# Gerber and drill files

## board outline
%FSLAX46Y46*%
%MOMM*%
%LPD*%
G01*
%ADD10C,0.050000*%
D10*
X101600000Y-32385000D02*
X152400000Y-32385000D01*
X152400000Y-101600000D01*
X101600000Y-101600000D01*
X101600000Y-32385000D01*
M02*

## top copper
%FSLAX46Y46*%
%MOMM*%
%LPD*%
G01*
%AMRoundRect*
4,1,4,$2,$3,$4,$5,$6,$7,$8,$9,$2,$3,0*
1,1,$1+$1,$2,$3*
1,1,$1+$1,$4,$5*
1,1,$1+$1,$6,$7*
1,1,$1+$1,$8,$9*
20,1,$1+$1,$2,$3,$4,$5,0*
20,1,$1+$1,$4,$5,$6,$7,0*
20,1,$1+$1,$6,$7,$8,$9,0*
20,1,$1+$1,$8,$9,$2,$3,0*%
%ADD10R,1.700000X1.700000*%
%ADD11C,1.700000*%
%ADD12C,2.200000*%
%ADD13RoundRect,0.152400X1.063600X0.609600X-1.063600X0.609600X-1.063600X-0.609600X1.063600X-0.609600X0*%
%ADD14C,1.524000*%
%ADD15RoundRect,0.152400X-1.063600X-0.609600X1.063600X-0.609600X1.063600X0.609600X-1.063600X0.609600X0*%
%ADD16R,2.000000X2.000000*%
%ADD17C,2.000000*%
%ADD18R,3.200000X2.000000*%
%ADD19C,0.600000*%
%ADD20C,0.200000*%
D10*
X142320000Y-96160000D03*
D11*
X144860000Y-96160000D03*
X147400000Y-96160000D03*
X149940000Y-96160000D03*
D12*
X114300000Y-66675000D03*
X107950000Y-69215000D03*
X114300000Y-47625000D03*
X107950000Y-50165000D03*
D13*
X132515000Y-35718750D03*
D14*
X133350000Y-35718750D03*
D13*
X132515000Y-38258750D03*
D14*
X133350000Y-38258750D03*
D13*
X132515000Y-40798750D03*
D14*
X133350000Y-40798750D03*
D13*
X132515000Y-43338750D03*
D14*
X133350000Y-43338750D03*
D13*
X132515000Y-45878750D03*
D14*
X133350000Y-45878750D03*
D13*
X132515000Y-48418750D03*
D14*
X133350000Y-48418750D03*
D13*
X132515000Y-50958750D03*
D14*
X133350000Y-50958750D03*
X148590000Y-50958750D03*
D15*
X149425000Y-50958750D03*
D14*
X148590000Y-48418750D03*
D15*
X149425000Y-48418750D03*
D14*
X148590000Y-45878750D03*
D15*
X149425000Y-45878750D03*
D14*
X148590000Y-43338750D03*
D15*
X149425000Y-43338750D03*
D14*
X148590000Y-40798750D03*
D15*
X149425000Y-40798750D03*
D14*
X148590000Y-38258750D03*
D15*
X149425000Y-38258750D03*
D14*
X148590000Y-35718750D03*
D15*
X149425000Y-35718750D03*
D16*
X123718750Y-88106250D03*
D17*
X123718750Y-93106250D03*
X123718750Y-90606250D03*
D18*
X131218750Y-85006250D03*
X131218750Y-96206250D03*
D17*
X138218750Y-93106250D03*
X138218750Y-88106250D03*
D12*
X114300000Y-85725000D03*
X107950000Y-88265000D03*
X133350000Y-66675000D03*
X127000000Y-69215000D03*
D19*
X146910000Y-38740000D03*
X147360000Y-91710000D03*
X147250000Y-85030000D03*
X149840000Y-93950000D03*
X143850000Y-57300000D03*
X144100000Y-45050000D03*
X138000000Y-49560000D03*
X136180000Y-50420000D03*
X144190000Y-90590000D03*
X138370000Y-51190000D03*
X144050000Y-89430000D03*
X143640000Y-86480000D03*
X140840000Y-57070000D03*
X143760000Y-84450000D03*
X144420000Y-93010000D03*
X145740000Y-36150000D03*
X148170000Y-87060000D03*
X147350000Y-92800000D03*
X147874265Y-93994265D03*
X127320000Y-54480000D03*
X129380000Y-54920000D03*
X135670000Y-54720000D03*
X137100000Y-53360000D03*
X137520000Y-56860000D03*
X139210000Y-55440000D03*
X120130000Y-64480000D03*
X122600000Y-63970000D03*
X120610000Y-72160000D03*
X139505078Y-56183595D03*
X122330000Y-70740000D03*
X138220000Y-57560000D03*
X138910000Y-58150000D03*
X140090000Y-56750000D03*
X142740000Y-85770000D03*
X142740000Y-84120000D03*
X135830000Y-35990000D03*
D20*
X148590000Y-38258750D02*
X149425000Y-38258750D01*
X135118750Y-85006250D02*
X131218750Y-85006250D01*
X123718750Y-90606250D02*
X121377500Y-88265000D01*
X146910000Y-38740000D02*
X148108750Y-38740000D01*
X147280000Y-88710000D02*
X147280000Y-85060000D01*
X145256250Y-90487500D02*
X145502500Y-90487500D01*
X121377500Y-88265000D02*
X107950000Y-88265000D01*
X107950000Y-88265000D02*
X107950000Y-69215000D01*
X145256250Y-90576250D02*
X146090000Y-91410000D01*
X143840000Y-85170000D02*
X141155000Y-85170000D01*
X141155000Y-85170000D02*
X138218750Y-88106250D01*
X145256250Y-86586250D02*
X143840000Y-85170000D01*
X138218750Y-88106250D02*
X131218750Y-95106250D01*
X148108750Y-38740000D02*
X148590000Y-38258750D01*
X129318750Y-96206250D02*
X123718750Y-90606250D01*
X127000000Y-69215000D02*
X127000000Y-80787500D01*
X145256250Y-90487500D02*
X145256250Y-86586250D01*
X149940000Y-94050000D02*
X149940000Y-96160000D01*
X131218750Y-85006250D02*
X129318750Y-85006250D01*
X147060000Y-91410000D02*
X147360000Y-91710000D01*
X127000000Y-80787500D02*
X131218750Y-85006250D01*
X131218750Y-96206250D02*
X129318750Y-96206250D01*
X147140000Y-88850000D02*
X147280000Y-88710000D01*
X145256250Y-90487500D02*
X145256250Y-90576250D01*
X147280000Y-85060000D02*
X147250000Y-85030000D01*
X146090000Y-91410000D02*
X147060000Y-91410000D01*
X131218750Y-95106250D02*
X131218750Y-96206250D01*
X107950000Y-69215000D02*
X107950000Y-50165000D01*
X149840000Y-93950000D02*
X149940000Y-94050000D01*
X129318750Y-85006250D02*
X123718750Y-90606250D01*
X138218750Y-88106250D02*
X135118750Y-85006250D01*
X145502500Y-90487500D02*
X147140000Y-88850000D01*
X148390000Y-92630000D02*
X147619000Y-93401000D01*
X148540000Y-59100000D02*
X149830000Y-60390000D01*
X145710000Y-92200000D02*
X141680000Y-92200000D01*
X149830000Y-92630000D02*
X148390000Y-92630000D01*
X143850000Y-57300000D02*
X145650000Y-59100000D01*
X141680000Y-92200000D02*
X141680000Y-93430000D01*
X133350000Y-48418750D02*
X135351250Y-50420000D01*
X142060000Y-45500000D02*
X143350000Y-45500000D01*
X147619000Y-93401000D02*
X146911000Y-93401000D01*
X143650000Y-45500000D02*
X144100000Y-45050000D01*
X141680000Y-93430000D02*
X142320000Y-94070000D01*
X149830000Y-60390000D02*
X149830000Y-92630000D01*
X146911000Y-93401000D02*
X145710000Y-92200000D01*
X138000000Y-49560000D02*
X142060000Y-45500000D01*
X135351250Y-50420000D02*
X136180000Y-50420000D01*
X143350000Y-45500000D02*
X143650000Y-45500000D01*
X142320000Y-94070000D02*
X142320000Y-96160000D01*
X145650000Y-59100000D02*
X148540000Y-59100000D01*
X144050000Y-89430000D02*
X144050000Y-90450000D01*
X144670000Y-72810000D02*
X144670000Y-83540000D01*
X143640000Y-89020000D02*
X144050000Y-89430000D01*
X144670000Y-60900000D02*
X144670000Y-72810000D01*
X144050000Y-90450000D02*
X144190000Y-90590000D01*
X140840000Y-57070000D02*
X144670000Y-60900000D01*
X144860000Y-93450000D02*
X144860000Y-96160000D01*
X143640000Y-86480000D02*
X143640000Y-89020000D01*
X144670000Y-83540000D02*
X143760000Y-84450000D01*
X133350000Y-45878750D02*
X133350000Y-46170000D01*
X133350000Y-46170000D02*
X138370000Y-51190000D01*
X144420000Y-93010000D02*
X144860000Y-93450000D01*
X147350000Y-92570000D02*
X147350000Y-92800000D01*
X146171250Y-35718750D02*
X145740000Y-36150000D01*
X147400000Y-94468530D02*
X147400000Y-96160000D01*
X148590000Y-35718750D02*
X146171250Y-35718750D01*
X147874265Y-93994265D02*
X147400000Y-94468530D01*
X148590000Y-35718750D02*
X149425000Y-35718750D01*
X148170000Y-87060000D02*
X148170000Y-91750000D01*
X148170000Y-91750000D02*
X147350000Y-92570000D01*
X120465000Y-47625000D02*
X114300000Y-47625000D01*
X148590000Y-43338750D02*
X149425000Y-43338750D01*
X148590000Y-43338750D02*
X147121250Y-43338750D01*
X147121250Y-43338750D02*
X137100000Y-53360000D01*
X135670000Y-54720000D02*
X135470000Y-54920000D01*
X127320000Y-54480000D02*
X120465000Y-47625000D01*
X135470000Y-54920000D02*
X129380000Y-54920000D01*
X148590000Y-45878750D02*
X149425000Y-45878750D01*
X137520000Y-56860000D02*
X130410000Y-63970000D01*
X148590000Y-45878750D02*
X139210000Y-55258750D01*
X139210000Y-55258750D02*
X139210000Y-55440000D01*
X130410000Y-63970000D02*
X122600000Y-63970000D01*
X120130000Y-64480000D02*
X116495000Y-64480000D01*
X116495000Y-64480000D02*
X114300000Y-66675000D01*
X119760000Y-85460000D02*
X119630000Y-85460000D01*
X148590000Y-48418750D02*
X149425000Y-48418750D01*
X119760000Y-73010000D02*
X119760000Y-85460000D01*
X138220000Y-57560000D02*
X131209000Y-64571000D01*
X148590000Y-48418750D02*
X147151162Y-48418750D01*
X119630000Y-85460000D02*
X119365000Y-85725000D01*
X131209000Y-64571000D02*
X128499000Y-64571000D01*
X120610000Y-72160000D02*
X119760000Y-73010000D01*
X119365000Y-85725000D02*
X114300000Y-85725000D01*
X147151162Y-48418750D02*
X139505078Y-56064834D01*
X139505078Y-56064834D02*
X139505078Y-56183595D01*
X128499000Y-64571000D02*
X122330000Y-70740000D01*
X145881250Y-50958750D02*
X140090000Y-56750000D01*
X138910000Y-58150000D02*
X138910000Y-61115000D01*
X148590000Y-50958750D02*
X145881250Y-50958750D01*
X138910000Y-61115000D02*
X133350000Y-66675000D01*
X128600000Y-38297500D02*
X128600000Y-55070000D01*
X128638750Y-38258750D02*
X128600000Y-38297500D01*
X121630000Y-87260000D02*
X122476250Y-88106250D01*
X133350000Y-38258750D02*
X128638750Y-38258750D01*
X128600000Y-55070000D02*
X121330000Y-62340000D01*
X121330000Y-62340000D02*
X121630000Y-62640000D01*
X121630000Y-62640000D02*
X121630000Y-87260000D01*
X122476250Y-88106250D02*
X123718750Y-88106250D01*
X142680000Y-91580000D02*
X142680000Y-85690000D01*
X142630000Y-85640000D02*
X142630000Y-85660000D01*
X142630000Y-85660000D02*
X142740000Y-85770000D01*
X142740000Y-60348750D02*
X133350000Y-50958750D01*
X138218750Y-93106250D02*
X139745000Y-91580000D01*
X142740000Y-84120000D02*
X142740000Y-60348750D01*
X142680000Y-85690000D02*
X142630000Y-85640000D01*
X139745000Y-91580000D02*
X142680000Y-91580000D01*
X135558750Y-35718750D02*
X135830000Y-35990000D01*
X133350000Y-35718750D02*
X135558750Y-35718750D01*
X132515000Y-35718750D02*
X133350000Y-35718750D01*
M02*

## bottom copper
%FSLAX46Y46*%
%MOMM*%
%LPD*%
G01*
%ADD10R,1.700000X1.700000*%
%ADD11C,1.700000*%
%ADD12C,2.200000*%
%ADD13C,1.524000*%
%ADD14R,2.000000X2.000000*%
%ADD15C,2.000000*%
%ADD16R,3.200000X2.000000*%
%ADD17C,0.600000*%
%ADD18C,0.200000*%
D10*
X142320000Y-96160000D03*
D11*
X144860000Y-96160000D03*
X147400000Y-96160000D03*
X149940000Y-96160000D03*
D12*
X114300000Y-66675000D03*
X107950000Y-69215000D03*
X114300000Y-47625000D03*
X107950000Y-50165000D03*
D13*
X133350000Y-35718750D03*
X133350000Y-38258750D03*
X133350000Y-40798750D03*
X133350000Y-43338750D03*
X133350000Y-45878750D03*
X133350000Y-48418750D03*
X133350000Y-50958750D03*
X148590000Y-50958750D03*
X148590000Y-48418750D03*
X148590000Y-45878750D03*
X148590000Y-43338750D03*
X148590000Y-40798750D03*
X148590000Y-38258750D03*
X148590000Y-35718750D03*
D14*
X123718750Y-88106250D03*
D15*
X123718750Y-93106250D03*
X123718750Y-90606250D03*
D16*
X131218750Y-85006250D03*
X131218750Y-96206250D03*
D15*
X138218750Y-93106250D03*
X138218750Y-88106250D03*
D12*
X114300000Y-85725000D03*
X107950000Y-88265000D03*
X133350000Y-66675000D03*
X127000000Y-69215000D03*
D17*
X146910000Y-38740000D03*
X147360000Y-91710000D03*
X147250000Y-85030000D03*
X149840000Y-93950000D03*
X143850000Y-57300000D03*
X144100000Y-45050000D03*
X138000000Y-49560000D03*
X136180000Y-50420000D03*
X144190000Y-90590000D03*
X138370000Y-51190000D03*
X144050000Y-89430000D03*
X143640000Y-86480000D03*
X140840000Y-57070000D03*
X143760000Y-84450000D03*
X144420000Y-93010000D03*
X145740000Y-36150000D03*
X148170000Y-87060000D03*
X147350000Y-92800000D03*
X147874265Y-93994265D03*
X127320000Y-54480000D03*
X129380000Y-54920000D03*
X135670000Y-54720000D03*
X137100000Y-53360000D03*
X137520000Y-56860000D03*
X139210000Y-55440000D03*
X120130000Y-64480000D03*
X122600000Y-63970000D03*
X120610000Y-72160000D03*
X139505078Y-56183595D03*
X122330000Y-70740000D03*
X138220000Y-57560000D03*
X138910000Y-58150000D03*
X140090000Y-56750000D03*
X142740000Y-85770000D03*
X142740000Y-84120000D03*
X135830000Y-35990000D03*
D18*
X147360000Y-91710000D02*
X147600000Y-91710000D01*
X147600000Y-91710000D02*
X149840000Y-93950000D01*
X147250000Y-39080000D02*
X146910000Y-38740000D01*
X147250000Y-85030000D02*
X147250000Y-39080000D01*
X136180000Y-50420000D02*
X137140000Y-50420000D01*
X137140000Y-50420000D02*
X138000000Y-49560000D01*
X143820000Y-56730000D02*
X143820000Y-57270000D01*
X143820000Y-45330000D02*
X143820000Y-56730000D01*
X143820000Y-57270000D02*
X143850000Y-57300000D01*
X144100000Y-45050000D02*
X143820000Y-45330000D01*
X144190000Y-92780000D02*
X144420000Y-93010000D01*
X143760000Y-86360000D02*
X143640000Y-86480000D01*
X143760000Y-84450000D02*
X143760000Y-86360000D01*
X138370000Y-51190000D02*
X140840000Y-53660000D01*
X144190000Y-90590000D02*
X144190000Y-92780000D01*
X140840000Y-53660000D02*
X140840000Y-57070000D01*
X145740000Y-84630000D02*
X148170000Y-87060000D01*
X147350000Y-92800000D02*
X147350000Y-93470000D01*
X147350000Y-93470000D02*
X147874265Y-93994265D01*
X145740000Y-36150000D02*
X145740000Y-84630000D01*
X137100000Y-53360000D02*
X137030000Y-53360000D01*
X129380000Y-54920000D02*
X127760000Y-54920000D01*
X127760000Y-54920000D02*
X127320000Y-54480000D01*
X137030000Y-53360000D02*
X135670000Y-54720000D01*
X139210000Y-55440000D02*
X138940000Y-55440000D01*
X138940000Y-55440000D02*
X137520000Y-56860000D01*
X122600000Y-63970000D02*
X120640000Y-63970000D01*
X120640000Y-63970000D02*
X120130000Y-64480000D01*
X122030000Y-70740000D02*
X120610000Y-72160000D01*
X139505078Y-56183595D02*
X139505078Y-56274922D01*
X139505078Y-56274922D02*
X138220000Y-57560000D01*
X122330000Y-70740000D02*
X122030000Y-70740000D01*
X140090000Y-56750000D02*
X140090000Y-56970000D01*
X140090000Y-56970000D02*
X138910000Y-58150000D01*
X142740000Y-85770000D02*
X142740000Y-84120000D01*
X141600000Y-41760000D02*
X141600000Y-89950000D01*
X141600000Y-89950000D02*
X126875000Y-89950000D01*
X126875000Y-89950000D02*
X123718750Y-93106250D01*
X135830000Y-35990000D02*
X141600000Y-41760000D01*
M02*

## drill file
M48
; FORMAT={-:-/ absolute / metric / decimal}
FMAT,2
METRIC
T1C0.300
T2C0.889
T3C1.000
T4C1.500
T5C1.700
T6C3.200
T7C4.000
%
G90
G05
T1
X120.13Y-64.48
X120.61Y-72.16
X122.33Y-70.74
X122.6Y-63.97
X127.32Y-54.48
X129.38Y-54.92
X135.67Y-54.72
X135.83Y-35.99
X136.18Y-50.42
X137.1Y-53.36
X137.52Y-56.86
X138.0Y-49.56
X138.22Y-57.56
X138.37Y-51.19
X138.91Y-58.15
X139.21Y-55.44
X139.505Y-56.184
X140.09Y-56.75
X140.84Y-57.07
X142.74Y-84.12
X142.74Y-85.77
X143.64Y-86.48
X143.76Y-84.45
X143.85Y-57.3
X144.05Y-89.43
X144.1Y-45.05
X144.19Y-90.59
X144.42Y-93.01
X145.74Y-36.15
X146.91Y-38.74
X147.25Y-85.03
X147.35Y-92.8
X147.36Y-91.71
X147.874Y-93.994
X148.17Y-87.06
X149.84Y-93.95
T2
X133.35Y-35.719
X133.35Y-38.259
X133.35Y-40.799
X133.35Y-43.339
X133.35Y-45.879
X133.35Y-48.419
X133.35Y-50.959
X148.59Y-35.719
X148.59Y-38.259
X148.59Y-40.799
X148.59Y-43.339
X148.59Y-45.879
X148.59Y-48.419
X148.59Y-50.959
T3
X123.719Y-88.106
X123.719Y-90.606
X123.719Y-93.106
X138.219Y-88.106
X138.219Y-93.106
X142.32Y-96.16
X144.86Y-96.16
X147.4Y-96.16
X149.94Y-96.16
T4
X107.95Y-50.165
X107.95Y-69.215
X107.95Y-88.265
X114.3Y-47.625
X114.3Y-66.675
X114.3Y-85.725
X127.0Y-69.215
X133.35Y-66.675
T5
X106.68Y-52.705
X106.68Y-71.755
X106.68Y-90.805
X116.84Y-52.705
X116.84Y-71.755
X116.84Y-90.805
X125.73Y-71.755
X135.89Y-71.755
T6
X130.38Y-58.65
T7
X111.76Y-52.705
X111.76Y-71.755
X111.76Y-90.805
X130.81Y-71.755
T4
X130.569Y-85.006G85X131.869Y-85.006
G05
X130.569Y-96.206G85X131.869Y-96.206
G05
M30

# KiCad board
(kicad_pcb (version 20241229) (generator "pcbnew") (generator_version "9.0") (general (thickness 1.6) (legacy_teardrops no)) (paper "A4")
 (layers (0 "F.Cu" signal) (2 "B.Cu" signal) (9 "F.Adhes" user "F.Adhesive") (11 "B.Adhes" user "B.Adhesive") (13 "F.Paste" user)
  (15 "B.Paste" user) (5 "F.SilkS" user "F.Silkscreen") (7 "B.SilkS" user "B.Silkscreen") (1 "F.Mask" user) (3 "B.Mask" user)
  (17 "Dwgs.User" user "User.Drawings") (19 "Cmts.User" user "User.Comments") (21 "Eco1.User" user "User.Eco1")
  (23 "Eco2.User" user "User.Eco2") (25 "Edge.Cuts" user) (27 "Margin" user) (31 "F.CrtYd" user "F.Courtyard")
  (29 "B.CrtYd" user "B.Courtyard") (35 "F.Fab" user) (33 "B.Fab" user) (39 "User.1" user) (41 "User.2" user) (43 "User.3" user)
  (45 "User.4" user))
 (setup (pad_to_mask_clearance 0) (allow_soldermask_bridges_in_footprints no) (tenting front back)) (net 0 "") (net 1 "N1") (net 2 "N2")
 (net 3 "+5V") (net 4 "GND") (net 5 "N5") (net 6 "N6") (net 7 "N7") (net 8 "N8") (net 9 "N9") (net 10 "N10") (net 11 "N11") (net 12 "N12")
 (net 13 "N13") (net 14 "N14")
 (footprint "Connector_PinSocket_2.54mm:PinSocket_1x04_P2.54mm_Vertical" (layer "F.Cu") (at 142.32 96.16 90)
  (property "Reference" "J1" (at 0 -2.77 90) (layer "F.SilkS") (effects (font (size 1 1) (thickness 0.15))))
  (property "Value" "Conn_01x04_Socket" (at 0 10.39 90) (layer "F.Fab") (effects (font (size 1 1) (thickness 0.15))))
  (pad "1" thru_hole rect (at 0 0 90) (size 1.7 1.7) (drill 1) (layers "*.Cu" "*.Mask") (remove_unused_layers no) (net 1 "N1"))
  (pad "2" thru_hole circle (at 0 2.54 90) (size 1.7 1.7) (drill 1) (layers "*.Cu" "*.Mask") (remove_unused_layers no) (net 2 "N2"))
  (pad "3" thru_hole circle (at 0 5.08 90) (size 1.7 1.7) (drill 1) (layers "*.Cu" "*.Mask") (remove_unused_layers no) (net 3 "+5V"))
  (pad "4" thru_hole circle (at 0 7.62 90) (size 1.7 1.7) (drill 1) (layers "*.Cu" "*.Mask") (remove_unused_layers no) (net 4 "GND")))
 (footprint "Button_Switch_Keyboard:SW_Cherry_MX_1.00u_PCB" (layer "F.Cu") (at 114.3 66.675)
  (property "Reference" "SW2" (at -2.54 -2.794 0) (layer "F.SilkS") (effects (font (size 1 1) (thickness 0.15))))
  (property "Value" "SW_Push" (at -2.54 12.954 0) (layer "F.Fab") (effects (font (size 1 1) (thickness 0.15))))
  (pad "" np_thru_hole circle (at -7.62 5.08) (size 1.7 1.7) (drill 1.7) (layers "*.Cu" "*.Mask"))
  (pad "" np_thru_hole circle (at -2.54 5.08) (size 4 4) (drill 4) (layers "*.Cu" "*.Mask"))
  (pad "" np_thru_hole circle (at 2.54 5.08) (size 1.7 1.7) (drill 1.7) (layers "*.Cu" "*.Mask"))
  (pad "1" thru_hole circle (at 0 0) (size 2.2 2.2) (drill 1.5) (layers "*.Cu" "*.Mask") (remove_unused_layers no) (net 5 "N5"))
  (pad "2" thru_hole circle (at -6.35 2.54) (size 2.2 2.2) (drill 1.5) (layers "*.Cu" "*.Mask") (remove_unused_layers no) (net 4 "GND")))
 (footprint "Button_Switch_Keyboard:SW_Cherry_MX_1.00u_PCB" (layer "F.Cu") (at 114.3 47.625)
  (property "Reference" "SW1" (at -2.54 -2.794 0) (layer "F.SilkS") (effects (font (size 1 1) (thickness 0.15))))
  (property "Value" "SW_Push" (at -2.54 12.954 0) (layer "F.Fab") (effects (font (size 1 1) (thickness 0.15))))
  (pad "" np_thru_hole circle (at -7.62 5.08) (size 1.7 1.7) (drill 1.7) (layers "*.Cu" "*.Mask"))
  (pad "" np_thru_hole circle (at -2.54 5.08) (size 4 4) (drill 4) (layers "*.Cu" "*.Mask"))
  (pad "" np_thru_hole circle (at 2.54 5.08) (size 1.7 1.7) (drill 1.7) (layers "*.Cu" "*.Mask"))
  (pad "1" thru_hole circle (at 0 0) (size 2.2 2.2) (drill 1.5) (layers "*.Cu" "*.Mask") (remove_unused_layers no) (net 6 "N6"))
  (pad "2" thru_hole circle (at -6.35 2.54) (size 2.2 2.2) (drill 1.5) (layers "*.Cu" "*.Mask") (remove_unused_layers no) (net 4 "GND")))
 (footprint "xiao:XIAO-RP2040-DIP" (layer "F.Cu") (at 140.97 43.33875)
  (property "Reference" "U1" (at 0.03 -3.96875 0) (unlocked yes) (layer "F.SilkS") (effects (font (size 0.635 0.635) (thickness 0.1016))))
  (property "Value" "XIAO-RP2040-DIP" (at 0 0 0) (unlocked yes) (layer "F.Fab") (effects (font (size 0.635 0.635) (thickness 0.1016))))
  (pad "1" smd roundrect (at -8.455 -7.62 180) (size 2.432 1.524) (layers "F.Cu" "F.Mask") (roundrect_rratio 0.1) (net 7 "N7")
   (thermal_bridge_angle 45))
  (pad "1" thru_hole circle (at -7.62 -7.62 180) (size 1.524 1.524) (drill 0.889) (layers "*.Cu" "*.Mask") (remove_unused_layers no)
   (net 7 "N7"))
  (pad "2" smd roundrect (at -8.455 -5.08 180) (size 2.432 1.524) (layers "F.Cu" "F.Mask") (roundrect_rratio 0.1) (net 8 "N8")
   (thermal_bridge_angle 45))
  (pad "2" thru_hole circle (at -7.62 -5.08 180) (size 1.524 1.524) (drill 0.889) (layers "*.Cu" "*.Mask") (remove_unused_layers no)
   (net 8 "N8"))
  (pad "3" smd roundrect (at -8.455 -2.54 180) (size 2.432 1.524) (layers "F.Cu" "F.Mask") (roundrect_rratio 0.1) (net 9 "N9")
   (thermal_bridge_angle 45))
  (pad "3" thru_hole circle (at -7.62 -2.54 180) (size 1.524 1.524) (drill 0.889) (layers "*.Cu" "*.Mask") (remove_unused_layers no)
   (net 9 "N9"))
  (pad "4" smd roundrect (at -8.455 0 180) (size 2.432 1.524) (layers "F.Cu" "F.Mask") (roundrect_rratio 0.1) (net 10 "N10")
   (thermal_bridge_angle 45))
  (pad "4" thru_hole circle (at -7.62 0 180) (size 1.524 1.524) (drill 0.889) (layers "*.Cu" "*.Mask") (remove_unused_layers no)
   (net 10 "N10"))
  (pad "5" smd roundrect (at -8.455 2.54 180) (size 2.432 1.524) (layers "F.Cu" "F.Mask") (roundrect_rratio 0.1) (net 2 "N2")
   (thermal_bridge_angle 45))
  (pad "5" thru_hole circle (at -7.62 2.54 180) (size 1.524 1.524) (drill 0.889) (layers "*.Cu" "*.Mask") (remove_unused_layers no)
   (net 2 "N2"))
  (pad "6" smd roundrect (at -8.455 5.08 180) (size 2.432 1.524) (layers "F.Cu" "F.Mask") (roundrect_rratio 0.1) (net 1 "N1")
   (thermal_bridge_angle 45))
  (pad "6" thru_hole circle (at -7.62 5.08 180) (size 1.524 1.524) (drill 0.889) (layers "*.Cu" "*.Mask") (remove_unused_layers no)
   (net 1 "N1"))
  (pad "7" smd roundrect (at -8.455 7.62 180) (size 2.432 1.524) (layers "F.Cu" "F.Mask") (roundrect_rratio 0.1) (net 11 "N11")
   (thermal_bridge_angle 45))
  (pad "7" thru_hole circle (at -7.62 7.62 180) (size 1.524 1.524) (drill 0.889) (layers "*.Cu" "*.Mask") (remove_unused_layers no)
   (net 11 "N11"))
  (pad "8" thru_hole circle (at 7.62 7.62) (size 1.524 1.524) (drill 0.889) (layers "*.Cu" "*.Mask") (remove_unused_layers no)
   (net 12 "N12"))
  (pad "8" smd roundrect (at 8.455 7.62) (size 2.432 1.524) (layers "F.Cu" "F.Mask") (roundrect_rratio 0.1) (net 12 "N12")
   (thermal_bridge_angle 45))
  (pad "9" thru_hole circle (at 7.62 5.08) (size 1.524 1.524) (drill 0.889) (layers "*.Cu" "*.Mask") (remove_unused_layers no)
   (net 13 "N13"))
  (pad "9" smd roundrect (at 8.455 5.08) (size 2.432 1.524) (layers "F.Cu" "F.Mask") (roundrect_rratio 0.1) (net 13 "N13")
   (thermal_bridge_angle 45))
  (pad "10" thru_hole circle (at 7.62 2.54) (size 1.524 1.524) (drill 0.889) (layers "*.Cu" "*.Mask") (remove_unused_layers no) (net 5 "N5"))
  (pad "10" smd roundrect (at 8.455 2.54) (size 2.432 1.524) (layers "F.Cu" "F.Mask") (roundrect_rratio 0.1) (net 5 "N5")
   (thermal_bridge_angle 45))
  (pad "11" thru_hole circle (at 7.62 0) (size 1.524 1.524) (drill 0.889) (layers "*.Cu" "*.Mask") (remove_unused_layers no) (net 6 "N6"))
  (pad "11" smd roundrect (at 8.455 0) (size 2.432 1.524) (layers "F.Cu" "F.Mask") (roundrect_rratio 0.1) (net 6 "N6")
   (thermal_bridge_angle 45))
  (pad "12" thru_hole circle (at 7.62 -2.54) (size 1.524 1.524) (drill 0.889) (layers "*.Cu" "*.Mask") (remove_unused_layers no)
   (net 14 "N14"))
  (pad "12" smd roundrect (at 8.455 -2.54) (size 2.432 1.524) (layers "F.Cu" "F.Mask") (roundrect_rratio 0.1) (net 14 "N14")
   (thermal_bridge_angle 45))
  (pad "13" thru_hole circle (at 7.62 -5.08) (size 1.524 1.524) (drill 0.889) (layers "*.Cu" "*.Mask") (remove_unused_layers no)
   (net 4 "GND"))
  (pad "13" smd roundrect (at 8.455 -5.08) (size 2.432 1.524) (layers "F.Cu" "F.Mask") (roundrect_rratio 0.1) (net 4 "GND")
   (thermal_bridge_angle 45))
  (pad "14" thru_hole circle (at 7.62 -7.62) (size 1.524 1.524) (drill 0.889) (layers "*.Cu" "*.Mask") (remove_unused_layers no)
   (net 3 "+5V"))
  (pad "14" smd roundrect (at 8.455 -7.62) (size 2.432 1.524) (layers "F.Cu" "F.Mask") (roundrect_rratio 0.1) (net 3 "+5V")
   (thermal_bridge_angle 45)))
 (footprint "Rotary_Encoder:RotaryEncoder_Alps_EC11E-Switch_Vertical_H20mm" (layer "F.Cu") (at 123.71875 88.10625)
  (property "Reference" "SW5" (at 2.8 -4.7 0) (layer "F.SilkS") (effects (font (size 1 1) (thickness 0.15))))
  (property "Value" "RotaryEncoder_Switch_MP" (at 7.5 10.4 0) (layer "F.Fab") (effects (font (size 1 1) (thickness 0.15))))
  (pad "A" thru_hole rect (at 0 0) (size 2 2) (drill 1) (layers "*.Cu" "*.Mask") (remove_unused_layers no) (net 8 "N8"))
  (pad "B" thru_hole circle (at 0 5) (size 2 2) (drill 1) (layers "*.Cu" "*.Mask") (remove_unused_layers no) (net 7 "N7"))
  (pad "C" thru_hole circle (at 0 2.5) (size 2 2) (drill 1) (layers "*.Cu" "*.Mask") (remove_unused_layers no) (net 4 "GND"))
  (pad "MP" thru_hole rect (at 7.5 -3.1) (size 3.2 2) (drill oval 2.8 1.5) (layers "*.Cu" "*.Mask") (remove_unused_layers no) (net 4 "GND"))
  (pad "MP" thru_hole rect (at 7.5 8.1) (size 3.2 2) (drill oval 2.8 1.5) (layers "*.Cu" "*.Mask") (remove_unused_layers no) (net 4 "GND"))
  (pad "S1" thru_hole circle (at 14.5 5) (size 2 2) (drill 1) (layers "*.Cu" "*.Mask") (remove_unused_layers no) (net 11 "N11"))
  (pad "S2" thru_hole circle (at 14.5 0) (size 2 2) (drill 1) (layers "*.Cu" "*.Mask") (remove_unused_layers no) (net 4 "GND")))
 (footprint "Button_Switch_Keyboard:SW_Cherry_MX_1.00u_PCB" (layer "F.Cu") (at 114.3 85.725)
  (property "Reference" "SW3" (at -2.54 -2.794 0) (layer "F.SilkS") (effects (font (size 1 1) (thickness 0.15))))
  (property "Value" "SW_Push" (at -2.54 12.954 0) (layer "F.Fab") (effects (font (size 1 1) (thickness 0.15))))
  (pad "" np_thru_hole circle (at -7.62 5.08) (size 1.7 1.7) (drill 1.7) (layers "*.Cu" "*.Mask"))
  (pad "" np_thru_hole circle (at -2.54 5.08) (size 4 4) (drill 4) (layers "*.Cu" "*.Mask"))
  (pad "" np_thru_hole circle (at 2.54 5.08) (size 1.7 1.7) (drill 1.7) (layers "*.Cu" "*.Mask"))
  (pad "1" thru_hole circle (at 0 0) (size 2.2 2.2) (drill 1.5) (layers "*.Cu" "*.Mask") (remove_unused_layers no) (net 13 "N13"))
  (pad "2" thru_hole circle (at -6.35 2.54) (size 2.2 2.2) (drill 1.5) (layers "*.Cu" "*.Mask") (remove_unused_layers no) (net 4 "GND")))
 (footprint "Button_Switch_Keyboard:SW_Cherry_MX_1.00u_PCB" (layer "F.Cu") (at 133.35 66.675)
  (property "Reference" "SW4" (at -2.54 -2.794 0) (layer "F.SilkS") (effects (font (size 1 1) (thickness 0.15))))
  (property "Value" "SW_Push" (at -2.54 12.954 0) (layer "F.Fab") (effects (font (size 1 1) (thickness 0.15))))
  (pad "" np_thru_hole circle (at -7.62 5.08) (size 1.7 1.7) (drill 1.7) (layers "*.Cu" "*.Mask"))
  (pad "" np_thru_hole circle (at -2.54 5.08) (size 4 4) (drill 4) (layers "*.Cu" "*.Mask"))
  (pad "" np_thru_hole circle (at 2.54 5.08) (size 1.7 1.7) (drill 1.7) (layers "*.Cu" "*.Mask"))
  (pad "1" thru_hole circle (at 0 0) (size 2.2 2.2) (drill 1.5) (layers "*.Cu" "*.Mask") (remove_unused_layers no) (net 12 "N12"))
  (pad "2" thru_hole circle (at -6.35 2.54) (size 2.2 2.2) (drill 1.5) (layers "*.Cu" "*.Mask") (remove_unused_layers no) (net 4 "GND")))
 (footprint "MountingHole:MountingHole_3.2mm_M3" (layer "F.Cu") (at 130.38 58.65)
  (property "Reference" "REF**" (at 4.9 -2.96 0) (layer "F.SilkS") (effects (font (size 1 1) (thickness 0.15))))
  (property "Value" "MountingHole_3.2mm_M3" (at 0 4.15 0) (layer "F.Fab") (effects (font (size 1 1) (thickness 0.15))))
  (pad "" np_thru_hole circle (at 0 0) (size 3.2 3.2) (drill 3.2) (layers "*.Cu" "*.Mask")))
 (gr_rect (start 101.6 32.385) (end 152.4 101.6) (stroke (width 0.05) (type default)) (fill no) (layer "Edge.Cuts"))
 (segment (start 148.59 38.25875) (end 149.425 38.25875) (width 0.2) (layer "F.Cu") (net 4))
 (segment (start 135.11875 85.00625) (end 131.21875 85.00625) (width 0.2) (layer "F.Cu") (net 4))
 (segment (start 123.71875 90.60625) (end 121.3775 88.265) (width 0.2) (layer "F.Cu") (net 4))
 (segment (start 146.91 38.74) (end 148.10875 38.74) (width 0.2) (layer "F.Cu") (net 4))
 (segment (start 147.28 88.71) (end 147.28 85.06) (width 0.2) (layer "F.Cu") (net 4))
 (segment (start 145.25625 90.4875) (end 145.5025 90.4875) (width 0.2) (layer "F.Cu") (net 4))
 (segment (start 121.3775 88.265) (end 107.95 88.265) (width 0.2) (layer "F.Cu") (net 4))
 (segment (start 107.95 88.265) (end 107.95 69.215) (width 0.2) (layer "F.Cu") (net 4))
 (segment (start 145.25625 90.57625) (end 146.09 91.41) (width 0.2) (layer "F.Cu") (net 4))
 (segment (start 143.84 85.17) (end 141.155 85.17) (width 0.2) (layer "F.Cu") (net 4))
 (segment (start 141.155 85.17) (end 138.21875 88.10625) (width 0.2) (layer "F.Cu") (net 4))
 (segment (start 145.25625 86.58625) (end 143.84 85.17) (width 0.2) (layer "F.Cu") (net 4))
 (segment (start 138.21875 88.10625) (end 131.21875 95.10625) (width 0.2) (layer "F.Cu") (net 4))
 (segment (start 148.10875 38.74) (end 148.59 38.25875) (width 0.2) (layer "F.Cu") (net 4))
 (segment (start 129.31875 96.20625) (end 123.71875 90.60625) (width 0.2) (layer "F.Cu") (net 4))
 (segment (start 127 69.215) (end 127 80.7875) (width 0.2) (layer "F.Cu") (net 4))
 (segment (start 145.25625 90.4875) (end 145.25625 86.58625) (width 0.2) (layer "F.Cu") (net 4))
 (segment (start 149.94 94.05) (end 149.94 96.16) (width 0.2) (layer "F.Cu") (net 4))
 (segment (start 131.21875 85.00625) (end 129.31875 85.00625) (width 0.2) (layer "F.Cu") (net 4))
 (segment (start 147.06 91.41) (end 147.36 91.71) (width 0.2) (layer "F.Cu") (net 4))
 (segment (start 127 80.7875) (end 131.21875 85.00625) (width 0.2) (layer "F.Cu") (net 4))
 (segment (start 131.21875 96.20625) (end 129.31875 96.20625) (width 0.2) (layer "F.Cu") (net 4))
 (segment (start 147.14 88.85) (end 147.28 88.71) (width 0.2) (layer "F.Cu") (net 4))
 (segment (start 145.25625 90.4875) (end 145.25625 90.57625) (width 0.2) (layer "F.Cu") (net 4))
 (segment (start 147.28 85.06) (end 147.25 85.03) (width 0.2) (layer "F.Cu") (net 4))
 (segment (start 146.09 91.41) (end 147.06 91.41) (width 0.2) (layer "F.Cu") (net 4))
 (segment (start 131.21875 95.10625) (end 131.21875 96.20625) (width 0.2) (layer "F.Cu") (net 4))
 (segment (start 107.95 69.215) (end 107.95 50.165) (width 0.2) (layer "F.Cu") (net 4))
 (segment (start 149.84 93.95) (end 149.94 94.05) (width 0.2) (layer "F.Cu") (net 4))
 (segment (start 129.31875 85.00625) (end 123.71875 90.60625) (width 0.2) (layer "F.Cu") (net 4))
 (segment (start 138.21875 88.10625) (end 135.11875 85.00625) (width 0.2) (layer "F.Cu") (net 4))
 (segment (start 145.5025 90.4875) (end 147.14 88.85) (width 0.2) (layer "F.Cu") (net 4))
 (via (at 146.91 38.74) (size 0.6) (drill 0.3) (layers "F.Cu" "B.Cu") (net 4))
 (via (at 147.36 91.71) (size 0.6) (drill 0.3) (layers "F.Cu" "B.Cu") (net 4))
 (via (at 147.25 85.03) (size 0.6) (drill 0.3) (layers "F.Cu" "B.Cu") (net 4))
 (via (at 149.84 93.95) (size 0.6) (drill 0.3) (layers "F.Cu" "B.Cu") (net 4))
 (segment (start 147.36 91.71) (end 147.6 91.71) (width 0.2) (layer "B.Cu") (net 4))
 (segment (start 147.6 91.71) (end 149.84 93.95) (width 0.2) (layer "B.Cu") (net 4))
 (segment (start 147.25 39.08) (end 146.91 38.74) (width 0.2) (layer "B.Cu") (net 4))
 (segment (start 147.25 85.03) (end 147.25 39.08) (width 0.2) (layer "B.Cu") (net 4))
 (segment (start 148.39 92.63) (end 147.619 93.401) (width 0.2) (layer "F.Cu") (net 1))
 (segment (start 148.54 59.1) (end 149.83 60.39) (width 0.2) (layer "F.Cu") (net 1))
 (segment (start 145.71 92.2) (end 141.68 92.2) (width 0.2) (layer "F.Cu") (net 1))
 (segment (start 149.83 92.63) (end 148.39 92.63) (width 0.2) (layer "F.Cu") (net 1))
 (segment (start 143.85 57.3) (end 145.65 59.1) (width 0.2) (layer "F.Cu") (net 1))
 (segment (start 141.68 92.2) (end 141.68 93.43) (width 0.2) (layer "F.Cu") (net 1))
 (segment (start 133.35 48.41875) (end 135.35125 50.42) (width 0.2) (layer "F.Cu") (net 1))
 (segment (start 142.06 45.5) (end 143.35 45.5) (width 0.2) (layer "F.Cu") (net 1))
 (segment (start 147.619 93.401) (end 146.911 93.401) (width 0.2) (layer "F.Cu") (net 1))
 (segment (start 143.65 45.5) (end 144.1 45.05) (width 0.2) (layer "F.Cu") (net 1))
 (segment (start 141.68 93.43) (end 142.32 94.07) (width 0.2) (layer "F.Cu") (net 1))
 (segment (start 149.83 60.39) (end 149.83 92.63) (width 0.2) (layer "F.Cu") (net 1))
 (segment (start 146.911 93.401) (end 145.71 92.2) (width 0.2) (layer "F.Cu") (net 1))
 (segment (start 138 49.56) (end 142.06 45.5) (width 0.2) (layer "F.Cu") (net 1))
 (segment (start 135.35125 50.42) (end 136.18 50.42) (width 0.2) (layer "F.Cu") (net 1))
 (segment (start 143.35 45.5) (end 143.65 45.5) (width 0.2) (layer "F.Cu") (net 1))
 (segment (start 142.32 94.07) (end 142.32 96.16) (width 0.2) (layer "F.Cu") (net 1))
 (segment (start 145.65 59.1) (end 148.54 59.1) (width 0.2) (layer "F.Cu") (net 1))
 (via (at 143.85 57.3) (size 0.6) (drill 0.3) (layers "F.Cu" "B.Cu") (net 1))
 (via (at 144.1 45.05) (size 0.6) (drill 0.3) (layers "F.Cu" "B.Cu") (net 1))
 (via (at 138 49.56) (size 0.6) (drill 0.3) (layers "F.Cu" "B.Cu") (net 1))
 (via (at 136.18 50.42) (size 0.6) (drill 0.3) (layers "F.Cu" "B.Cu") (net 1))
 (segment (start 136.18 50.42) (end 137.14 50.42) (width 0.2) (layer "B.Cu") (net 1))
 (segment (start 137.14 50.42) (end 138 49.56) (width 0.2) (layer "B.Cu") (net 1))
 (segment (start 143.82 56.73) (end 143.82 57.27) (width 0.2) (layer "B.Cu") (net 1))
 (segment (start 143.82 45.33) (end 143.82 56.73) (width 0.2) (layer "B.Cu") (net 1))
 (segment (start 143.82 57.27) (end 143.85 57.3) (width 0.2) (layer "B.Cu") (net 1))
 (segment (start 144.1 45.05) (end 143.82 45.33) (width 0.2) (layer "B.Cu") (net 1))
 (segment (start 144.05 89.43) (end 144.05 90.45) (width 0.2) (layer "F.Cu") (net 2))
 (segment (start 144.67 72.81) (end 144.67 83.54) (width 0.2) (layer "F.Cu") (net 2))
 (segment (start 143.64 89.02) (end 144.05 89.43) (width 0.2) (layer "F.Cu") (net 2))
 (segment (start 144.67 60.9) (end 144.67 72.81) (width 0.2) (layer "F.Cu") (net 2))
 (segment (start 144.05 90.45) (end 144.19 90.59) (width 0.2) (layer "F.Cu") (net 2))
 (segment (start 140.84 57.07) (end 144.67 60.9) (width 0.2) (layer "F.Cu") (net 2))
 (segment (start 144.86 93.45) (end 144.86 96.16) (width 0.2) (layer "F.Cu") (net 2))
 (segment (start 143.64 86.48) (end 143.64 89.02) (width 0.2) (layer "F.Cu") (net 2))
 (segment (start 144.67 83.54) (end 143.76 84.45) (width 0.2) (layer "F.Cu") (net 2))
 (segment (start 133.35 45.87875) (end 133.35 46.17) (width 0.2) (layer "F.Cu") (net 2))
 (segment (start 133.35 46.17) (end 138.37 51.19) (width 0.2) (layer "F.Cu") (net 2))
 (segment (start 144.42 93.01) (end 144.86 93.45) (width 0.2) (layer "F.Cu") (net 2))
 (via (at 144.19 90.59) (size 0.6) (drill 0.3) (layers "F.Cu" "B.Cu") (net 2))
 (via (at 138.37 51.19) (size 0.6) (drill 0.3) (layers "F.Cu" "B.Cu") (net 2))
 (via (at 144.05 89.43) (size 0.6) (drill 0.3) (layers "F.Cu" "B.Cu") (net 2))
 (via (at 143.64 86.48) (size 0.6) (drill 0.3) (layers "F.Cu" "B.Cu") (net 2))
 (via (at 140.84 57.07) (size 0.6) (drill 0.3) (layers "F.Cu" "B.Cu") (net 2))
 (via (at 143.76 84.45) (size 0.6) (drill 0.3) (layers "F.Cu" "B.Cu") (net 2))
 (via (at 144.42 93.01) (size 0.6) (drill 0.3) (layers "F.Cu" "B.Cu") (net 2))
 (segment (start 144.19 92.78) (end 144.42 93.01) (width 0.2) (layer "B.Cu") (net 2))
 (segment (start 143.76 86.36) (end 143.64 86.48) (width 0.2) (layer "B.Cu") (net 2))
 (segment (start 143.76 84.45) (end 143.76 86.36) (width 0.2) (layer "B.Cu") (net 2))
 (segment (start 138.37 51.19) (end 140.84 53.66) (width 0.2) (layer "B.Cu") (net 2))
 (segment (start 144.19 90.59) (end 144.19 92.78) (width 0.2) (layer "B.Cu") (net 2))
 (segment (start 140.84 53.66) (end 140.84 57.07) (width 0.2) (layer "B.Cu") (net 2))
 (segment (start 147.35 92.57) (end 147.35 92.8) (width 0.2) (layer "F.Cu") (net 3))
 (segment (start 146.17125 35.71875) (end 145.74 36.15) (width 0.2) (layer "F.Cu") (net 3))
 (segment (start 147.4 94.46853) (end 147.4 96.16) (width 0.2) (layer "F.Cu") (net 3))
 (segment (start 148.59 35.71875) (end 146.17125 35.71875) (width 0.2) (layer "F.Cu") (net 3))
 (segment (start 147.874265 93.994265) (end 147.4 94.46853) (width 0.2) (layer "F.Cu") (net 3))
 (segment (start 148.59 35.71875) (end 149.425 35.71875) (width 0.2) (layer "F.Cu") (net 3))
 (segment (start 148.17 87.06) (end 148.17 91.75) (width 0.2) (layer "F.Cu") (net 3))
 (segment (start 148.17 91.75) (end 147.35 92.57) (width 0.2) (layer "F.Cu") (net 3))
 (via (at 145.74 36.15) (size 0.6) (drill 0.3) (layers "F.Cu" "B.Cu") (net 3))
 (via (at 148.17 87.06) (size 0.6) (drill 0.3) (layers "F.Cu" "B.Cu") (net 3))
 (via (at 147.35 92.8) (size 0.6) (drill 0.3) (layers "F.Cu" "B.Cu") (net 3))
 (via (at 147.874265 93.994265) (size 0.6) (drill 0.3) (layers "F.Cu" "B.Cu") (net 3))
 (segment (start 145.74 84.63) (end 148.17 87.06) (width 0.2) (layer "B.Cu") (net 3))
 (segment (start 147.35 92.8) (end 147.35 93.47) (width 0.2) (layer "B.Cu") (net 3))
 (segment (start 147.35 93.47) (end 147.874265 93.994265) (width 0.2) (layer "B.Cu") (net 3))
 (segment (start 145.74 36.15) (end 145.74 84.63) (width 0.2) (layer "B.Cu") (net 3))
 (segment (start 120.465 47.625) (end 114.3 47.625) (width 0.2) (layer "F.Cu") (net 6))
 (segment (start 148.59 43.33875) (end 149.425 43.33875) (width 0.2) (layer "F.Cu") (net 6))
 (segment (start 148.59 43.33875) (end 147.12125 43.33875) (width 0.2) (layer "F.Cu") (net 6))
 (segment (start 147.12125 43.33875) (end 137.1 53.36) (width 0.2) (layer "F.Cu") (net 6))
 (segment (start 135.67 54.72) (end 135.47 54.92) (width 0.2) (layer "F.Cu") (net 6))
 (segment (start 127.32 54.48) (end 120.465 47.625) (width 0.2) (layer "F.Cu") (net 6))
 (segment (start 135.47 54.92) (end 129.38 54.92) (width 0.2) (layer "F.Cu") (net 6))
 (via (at 127.32 54.48) (size 0.6) (drill 0.3) (layers "F.Cu" "B.Cu") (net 6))
 (via (at 129.38 54.92) (size 0.6) (drill 0.3) (layers "F.Cu" "B.Cu") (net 6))
 (via (at 135.67 54.72) (size 0.6) (drill 0.3) (layers "F.Cu" "B.Cu") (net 6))
 (via (at 137.1 53.36) (size 0.6) (drill 0.3) (layers "F.Cu" "B.Cu") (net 6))
 (segment (start 137.1 53.36) (end 137.03 53.36) (width 0.2) (layer "B.Cu") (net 6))
 (segment (start 129.38 54.92) (end 127.76 54.92) (width 0.2) (layer "B.Cu") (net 6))
 (segment (start 127.76 54.92) (end 127.32 54.48) (width 0.2) (layer "B.Cu") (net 6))
 (segment (start 137.03 53.36) (end 135.67 54.72) (width 0.2) (layer "B.Cu") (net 6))
 (segment (start 148.59 45.87875) (end 149.425 45.87875) (width 0.2) (layer "F.Cu") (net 5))
 (segment (start 137.52 56.86) (end 130.41 63.97) (width 0.2) (layer "F.Cu") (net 5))
 (segment (start 148.59 45.87875) (end 139.21 55.25875) (width 0.2) (layer "F.Cu") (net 5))
 (segment (start 139.21 55.25875) (end 139.21 55.44) (width 0.2) (layer "F.Cu") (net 5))
 (segment (start 130.41 63.97) (end 122.6 63.97) (width 0.2) (layer "F.Cu") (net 5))
 (segment (start 120.13 64.48) (end 116.495 64.48) (width 0.2) (layer "F.Cu") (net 5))
 (segment (start 116.495 64.48) (end 114.3 66.675) (width 0.2) (layer "F.Cu") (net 5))
 (via (at 137.52 56.86) (size 0.6) (drill 0.3) (layers "F.Cu" "B.Cu") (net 5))
 (via (at 139.21 55.44) (size 0.6) (drill 0.3) (layers "F.Cu" "B.Cu") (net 5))
 (via (at 120.13 64.48) (size 0.6) (drill 0.3) (layers "F.Cu" "B.Cu") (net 5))
 (via (at 122.6 63.97) (size 0.6) (drill 0.3) (layers "F.Cu" "B.Cu") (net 5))
 (segment (start 139.21 55.44) (end 138.94 55.44) (width 0.2) (layer "B.Cu") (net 5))
 (segment (start 138.94 55.44) (end 137.52 56.86) (width 0.2) (layer "B.Cu") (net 5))
 (segment (start 122.6 63.97) (end 120.64 63.97) (width 0.2) (layer "B.Cu") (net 5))
 (segment (start 120.64 63.97) (end 120.13 64.48) (width 0.2) (layer "B.Cu") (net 5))
 (segment (start 119.76 85.46) (end 119.63 85.46) (width 0.2) (layer "F.Cu") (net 13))
 (segment (start 148.59 48.41875) (end 149.425 48.41875) (width 0.2) (layer "F.Cu") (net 13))
 (segment (start 119.76 73.01) (end 119.76 85.46) (width 0.2) (layer "F.Cu") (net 13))
 (segment (start 138.22 57.56) (end 131.209 64.571) (width 0.2) (layer "F.Cu") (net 13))
 (segment (start 148.59 48.41875) (end 147.151162 48.41875) (width 0.2) (layer "F.Cu") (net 13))
 (segment (start 119.63 85.46) (end 119.365 85.725) (width 0.2) (layer "F.Cu") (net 13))
 (segment (start 131.209 64.571) (end 128.499 64.571) (width 0.2) (layer "F.Cu") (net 13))
 (segment (start 120.61 72.16) (end 119.76 73.01) (width 0.2) (layer "F.Cu") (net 13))
 (segment (start 119.365 85.725) (end 114.3 85.725) (width 0.2) (layer "F.Cu") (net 13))
 (segment (start 147.151162 48.41875) (end 139.505078 56.064834) (width 0.2) (layer "F.Cu") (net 13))
 (segment (start 139.505078 56.064834) (end 139.505078 56.183595) (width 0.2) (layer "F.Cu") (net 13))
 (segment (start 128.499 64.571) (end 122.33 70.74) (width 0.2) (layer "F.Cu") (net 13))
 (via (at 120.61 72.16) (size 0.6) (drill 0.3) (layers "F.Cu" "B.Cu") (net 13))
 (via (at 139.505078 56.183595) (size 0.6) (drill 0.3) (layers "F.Cu" "B.Cu") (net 13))
 (via (at 122.33 70.74) (size 0.6) (drill 0.3) (layers "F.Cu" "B.Cu") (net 13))
 (via (at 138.22 57.56) (size 0.6) (drill 0.3) (layers "F.Cu" "B.Cu") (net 13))
 (segment (start 122.03 70.74) (end 120.61 72.16) (width 0.2) (layer "B.Cu") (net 13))
 (segment (start 139.505078 56.183595) (end 139.505078 56.274922) (width 0.2) (layer "B.Cu") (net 13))
 (segment (start 139.505078 56.274922) (end 138.22 57.56) (width 0.2) (layer "B.Cu") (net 13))
 (segment (start 122.33 70.74) (end 122.03 70.74) (width 0.2) (layer "B.Cu") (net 13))
 (segment (start 145.88125 50.95875) (end 140.09 56.75) (width 0.2) (layer "F.Cu") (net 12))
 (segment (start 138.91 58.15) (end 138.91 61.115) (width 0.2) (layer "F.Cu") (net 12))
 (segment (start 148.59 50.95875) (end 145.88125 50.95875) (width 0.2) (layer "F.Cu") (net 12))
 (segment (start 138.91 61.115) (end 133.35 66.675) (width 0.2) (layer "F.Cu") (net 12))
 (via (at 138.91 58.15) (size 0.6) (drill 0.3) (layers "F.Cu" "B.Cu") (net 12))
 (via (at 140.09 56.75) (size 0.6) (drill 0.3) (layers "F.Cu" "B.Cu") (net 12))
 (segment (start 140.09 56.75) (end 140.09 56.97) (width 0.2) (layer "B.Cu") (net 12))
 (segment (start 140.09 56.97) (end 138.91 58.15) (width 0.2) (layer "B.Cu") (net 12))
 (segment (start 128.6 38.2975) (end 128.6 55.07) (width 0.2) (layer "F.Cu") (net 8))
 (segment (start 128.63875 38.25875) (end 128.6 38.2975) (width 0.2) (layer "F.Cu") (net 8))
 (segment (start 121.63 87.26) (end 122.47625 88.10625) (width 0.2) (layer "F.Cu") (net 8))
 (segment (start 133.35 38.25875) (end 128.63875 38.25875) (width 0.2) (layer "F.Cu") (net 8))
 (segment (start 128.6 55.07) (end 121.33 62.34) (width 0.2) (layer "F.Cu") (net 8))
 (segment (start 121.33 62.34) (end 121.63 62.64) (width 0.2) (layer "F.Cu") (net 8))
 (segment (start 121.63 62.64) (end 121.63 87.26) (width 0.2) (layer "F.Cu") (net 8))
 (segment (start 122.47625 88.10625) (end 123.71875 88.10625) (width 0.2) (layer "F.Cu") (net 8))
 (segment (start 142.68 91.58) (end 142.68 85.69) (width 0.2) (layer "F.Cu") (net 11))
 (segment (start 142.63 85.64) (end 142.63 85.66) (width 0.2) (layer "F.Cu") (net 11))
 (segment (start 142.63 85.66) (end 142.74 85.77) (width 0.2) (layer "F.Cu") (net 11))
 (segment (start 142.74 60.34875) (end 133.35 50.95875) (width 0.2) (layer "F.Cu") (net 11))
 (segment (start 138.21875 93.10625) (end 139.745 91.58) (width 0.2) (layer "F.Cu") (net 11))
 (segment (start 142.74 84.12) (end 142.74 60.34875) (width 0.2) (layer "F.Cu") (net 11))
 (segment (start 142.68 85.69) (end 142.63 85.64) (width 0.2) (layer "F.Cu") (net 11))
 (segment (start 139.745 91.58) (end 142.68 91.58) (width 0.2) (layer "F.Cu") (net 11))
 (via (at 142.74 85.77) (size 0.6) (drill 0.3) (layers "F.Cu" "B.Cu") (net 11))
 (via (at 142.74 84.12) (size 0.6) (drill 0.3) (layers "F.Cu" "B.Cu") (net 11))
 (segment (start 142.74 85.77) (end 142.74 84.12) (width 0.2) (layer "B.Cu") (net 11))
 (segment (start 135.55875 35.71875) (end 135.83 35.99) (width 0.2) (layer "F.Cu") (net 7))
 (segment (start 133.35 35.71875) (end 135.55875 35.71875) (width 0.2) (layer "F.Cu") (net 7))
 (segment (start 132.515 35.71875) (end 133.35 35.71875) (width 0.2) (layer "F.Cu") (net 7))
 (via (at 135.83 35.99) (size 0.6) (drill 0.3) (layers "F.Cu" "B.Cu") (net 7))
 (segment (start 141.6 41.76) (end 141.6 89.95) (width 0.2) (layer "B.Cu") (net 7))
 (segment (start 141.6 89.95) (end 126.875 89.95) (width 0.2) (layer "B.Cu") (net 7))
 (segment (start 126.875 89.95) (end 123.71875 93.10625) (width 0.2) (layer "B.Cu") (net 7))
 (segment (start 135.83 35.99) (end 141.6 41.76) (width 0.2) (layer "B.Cu") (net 7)))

